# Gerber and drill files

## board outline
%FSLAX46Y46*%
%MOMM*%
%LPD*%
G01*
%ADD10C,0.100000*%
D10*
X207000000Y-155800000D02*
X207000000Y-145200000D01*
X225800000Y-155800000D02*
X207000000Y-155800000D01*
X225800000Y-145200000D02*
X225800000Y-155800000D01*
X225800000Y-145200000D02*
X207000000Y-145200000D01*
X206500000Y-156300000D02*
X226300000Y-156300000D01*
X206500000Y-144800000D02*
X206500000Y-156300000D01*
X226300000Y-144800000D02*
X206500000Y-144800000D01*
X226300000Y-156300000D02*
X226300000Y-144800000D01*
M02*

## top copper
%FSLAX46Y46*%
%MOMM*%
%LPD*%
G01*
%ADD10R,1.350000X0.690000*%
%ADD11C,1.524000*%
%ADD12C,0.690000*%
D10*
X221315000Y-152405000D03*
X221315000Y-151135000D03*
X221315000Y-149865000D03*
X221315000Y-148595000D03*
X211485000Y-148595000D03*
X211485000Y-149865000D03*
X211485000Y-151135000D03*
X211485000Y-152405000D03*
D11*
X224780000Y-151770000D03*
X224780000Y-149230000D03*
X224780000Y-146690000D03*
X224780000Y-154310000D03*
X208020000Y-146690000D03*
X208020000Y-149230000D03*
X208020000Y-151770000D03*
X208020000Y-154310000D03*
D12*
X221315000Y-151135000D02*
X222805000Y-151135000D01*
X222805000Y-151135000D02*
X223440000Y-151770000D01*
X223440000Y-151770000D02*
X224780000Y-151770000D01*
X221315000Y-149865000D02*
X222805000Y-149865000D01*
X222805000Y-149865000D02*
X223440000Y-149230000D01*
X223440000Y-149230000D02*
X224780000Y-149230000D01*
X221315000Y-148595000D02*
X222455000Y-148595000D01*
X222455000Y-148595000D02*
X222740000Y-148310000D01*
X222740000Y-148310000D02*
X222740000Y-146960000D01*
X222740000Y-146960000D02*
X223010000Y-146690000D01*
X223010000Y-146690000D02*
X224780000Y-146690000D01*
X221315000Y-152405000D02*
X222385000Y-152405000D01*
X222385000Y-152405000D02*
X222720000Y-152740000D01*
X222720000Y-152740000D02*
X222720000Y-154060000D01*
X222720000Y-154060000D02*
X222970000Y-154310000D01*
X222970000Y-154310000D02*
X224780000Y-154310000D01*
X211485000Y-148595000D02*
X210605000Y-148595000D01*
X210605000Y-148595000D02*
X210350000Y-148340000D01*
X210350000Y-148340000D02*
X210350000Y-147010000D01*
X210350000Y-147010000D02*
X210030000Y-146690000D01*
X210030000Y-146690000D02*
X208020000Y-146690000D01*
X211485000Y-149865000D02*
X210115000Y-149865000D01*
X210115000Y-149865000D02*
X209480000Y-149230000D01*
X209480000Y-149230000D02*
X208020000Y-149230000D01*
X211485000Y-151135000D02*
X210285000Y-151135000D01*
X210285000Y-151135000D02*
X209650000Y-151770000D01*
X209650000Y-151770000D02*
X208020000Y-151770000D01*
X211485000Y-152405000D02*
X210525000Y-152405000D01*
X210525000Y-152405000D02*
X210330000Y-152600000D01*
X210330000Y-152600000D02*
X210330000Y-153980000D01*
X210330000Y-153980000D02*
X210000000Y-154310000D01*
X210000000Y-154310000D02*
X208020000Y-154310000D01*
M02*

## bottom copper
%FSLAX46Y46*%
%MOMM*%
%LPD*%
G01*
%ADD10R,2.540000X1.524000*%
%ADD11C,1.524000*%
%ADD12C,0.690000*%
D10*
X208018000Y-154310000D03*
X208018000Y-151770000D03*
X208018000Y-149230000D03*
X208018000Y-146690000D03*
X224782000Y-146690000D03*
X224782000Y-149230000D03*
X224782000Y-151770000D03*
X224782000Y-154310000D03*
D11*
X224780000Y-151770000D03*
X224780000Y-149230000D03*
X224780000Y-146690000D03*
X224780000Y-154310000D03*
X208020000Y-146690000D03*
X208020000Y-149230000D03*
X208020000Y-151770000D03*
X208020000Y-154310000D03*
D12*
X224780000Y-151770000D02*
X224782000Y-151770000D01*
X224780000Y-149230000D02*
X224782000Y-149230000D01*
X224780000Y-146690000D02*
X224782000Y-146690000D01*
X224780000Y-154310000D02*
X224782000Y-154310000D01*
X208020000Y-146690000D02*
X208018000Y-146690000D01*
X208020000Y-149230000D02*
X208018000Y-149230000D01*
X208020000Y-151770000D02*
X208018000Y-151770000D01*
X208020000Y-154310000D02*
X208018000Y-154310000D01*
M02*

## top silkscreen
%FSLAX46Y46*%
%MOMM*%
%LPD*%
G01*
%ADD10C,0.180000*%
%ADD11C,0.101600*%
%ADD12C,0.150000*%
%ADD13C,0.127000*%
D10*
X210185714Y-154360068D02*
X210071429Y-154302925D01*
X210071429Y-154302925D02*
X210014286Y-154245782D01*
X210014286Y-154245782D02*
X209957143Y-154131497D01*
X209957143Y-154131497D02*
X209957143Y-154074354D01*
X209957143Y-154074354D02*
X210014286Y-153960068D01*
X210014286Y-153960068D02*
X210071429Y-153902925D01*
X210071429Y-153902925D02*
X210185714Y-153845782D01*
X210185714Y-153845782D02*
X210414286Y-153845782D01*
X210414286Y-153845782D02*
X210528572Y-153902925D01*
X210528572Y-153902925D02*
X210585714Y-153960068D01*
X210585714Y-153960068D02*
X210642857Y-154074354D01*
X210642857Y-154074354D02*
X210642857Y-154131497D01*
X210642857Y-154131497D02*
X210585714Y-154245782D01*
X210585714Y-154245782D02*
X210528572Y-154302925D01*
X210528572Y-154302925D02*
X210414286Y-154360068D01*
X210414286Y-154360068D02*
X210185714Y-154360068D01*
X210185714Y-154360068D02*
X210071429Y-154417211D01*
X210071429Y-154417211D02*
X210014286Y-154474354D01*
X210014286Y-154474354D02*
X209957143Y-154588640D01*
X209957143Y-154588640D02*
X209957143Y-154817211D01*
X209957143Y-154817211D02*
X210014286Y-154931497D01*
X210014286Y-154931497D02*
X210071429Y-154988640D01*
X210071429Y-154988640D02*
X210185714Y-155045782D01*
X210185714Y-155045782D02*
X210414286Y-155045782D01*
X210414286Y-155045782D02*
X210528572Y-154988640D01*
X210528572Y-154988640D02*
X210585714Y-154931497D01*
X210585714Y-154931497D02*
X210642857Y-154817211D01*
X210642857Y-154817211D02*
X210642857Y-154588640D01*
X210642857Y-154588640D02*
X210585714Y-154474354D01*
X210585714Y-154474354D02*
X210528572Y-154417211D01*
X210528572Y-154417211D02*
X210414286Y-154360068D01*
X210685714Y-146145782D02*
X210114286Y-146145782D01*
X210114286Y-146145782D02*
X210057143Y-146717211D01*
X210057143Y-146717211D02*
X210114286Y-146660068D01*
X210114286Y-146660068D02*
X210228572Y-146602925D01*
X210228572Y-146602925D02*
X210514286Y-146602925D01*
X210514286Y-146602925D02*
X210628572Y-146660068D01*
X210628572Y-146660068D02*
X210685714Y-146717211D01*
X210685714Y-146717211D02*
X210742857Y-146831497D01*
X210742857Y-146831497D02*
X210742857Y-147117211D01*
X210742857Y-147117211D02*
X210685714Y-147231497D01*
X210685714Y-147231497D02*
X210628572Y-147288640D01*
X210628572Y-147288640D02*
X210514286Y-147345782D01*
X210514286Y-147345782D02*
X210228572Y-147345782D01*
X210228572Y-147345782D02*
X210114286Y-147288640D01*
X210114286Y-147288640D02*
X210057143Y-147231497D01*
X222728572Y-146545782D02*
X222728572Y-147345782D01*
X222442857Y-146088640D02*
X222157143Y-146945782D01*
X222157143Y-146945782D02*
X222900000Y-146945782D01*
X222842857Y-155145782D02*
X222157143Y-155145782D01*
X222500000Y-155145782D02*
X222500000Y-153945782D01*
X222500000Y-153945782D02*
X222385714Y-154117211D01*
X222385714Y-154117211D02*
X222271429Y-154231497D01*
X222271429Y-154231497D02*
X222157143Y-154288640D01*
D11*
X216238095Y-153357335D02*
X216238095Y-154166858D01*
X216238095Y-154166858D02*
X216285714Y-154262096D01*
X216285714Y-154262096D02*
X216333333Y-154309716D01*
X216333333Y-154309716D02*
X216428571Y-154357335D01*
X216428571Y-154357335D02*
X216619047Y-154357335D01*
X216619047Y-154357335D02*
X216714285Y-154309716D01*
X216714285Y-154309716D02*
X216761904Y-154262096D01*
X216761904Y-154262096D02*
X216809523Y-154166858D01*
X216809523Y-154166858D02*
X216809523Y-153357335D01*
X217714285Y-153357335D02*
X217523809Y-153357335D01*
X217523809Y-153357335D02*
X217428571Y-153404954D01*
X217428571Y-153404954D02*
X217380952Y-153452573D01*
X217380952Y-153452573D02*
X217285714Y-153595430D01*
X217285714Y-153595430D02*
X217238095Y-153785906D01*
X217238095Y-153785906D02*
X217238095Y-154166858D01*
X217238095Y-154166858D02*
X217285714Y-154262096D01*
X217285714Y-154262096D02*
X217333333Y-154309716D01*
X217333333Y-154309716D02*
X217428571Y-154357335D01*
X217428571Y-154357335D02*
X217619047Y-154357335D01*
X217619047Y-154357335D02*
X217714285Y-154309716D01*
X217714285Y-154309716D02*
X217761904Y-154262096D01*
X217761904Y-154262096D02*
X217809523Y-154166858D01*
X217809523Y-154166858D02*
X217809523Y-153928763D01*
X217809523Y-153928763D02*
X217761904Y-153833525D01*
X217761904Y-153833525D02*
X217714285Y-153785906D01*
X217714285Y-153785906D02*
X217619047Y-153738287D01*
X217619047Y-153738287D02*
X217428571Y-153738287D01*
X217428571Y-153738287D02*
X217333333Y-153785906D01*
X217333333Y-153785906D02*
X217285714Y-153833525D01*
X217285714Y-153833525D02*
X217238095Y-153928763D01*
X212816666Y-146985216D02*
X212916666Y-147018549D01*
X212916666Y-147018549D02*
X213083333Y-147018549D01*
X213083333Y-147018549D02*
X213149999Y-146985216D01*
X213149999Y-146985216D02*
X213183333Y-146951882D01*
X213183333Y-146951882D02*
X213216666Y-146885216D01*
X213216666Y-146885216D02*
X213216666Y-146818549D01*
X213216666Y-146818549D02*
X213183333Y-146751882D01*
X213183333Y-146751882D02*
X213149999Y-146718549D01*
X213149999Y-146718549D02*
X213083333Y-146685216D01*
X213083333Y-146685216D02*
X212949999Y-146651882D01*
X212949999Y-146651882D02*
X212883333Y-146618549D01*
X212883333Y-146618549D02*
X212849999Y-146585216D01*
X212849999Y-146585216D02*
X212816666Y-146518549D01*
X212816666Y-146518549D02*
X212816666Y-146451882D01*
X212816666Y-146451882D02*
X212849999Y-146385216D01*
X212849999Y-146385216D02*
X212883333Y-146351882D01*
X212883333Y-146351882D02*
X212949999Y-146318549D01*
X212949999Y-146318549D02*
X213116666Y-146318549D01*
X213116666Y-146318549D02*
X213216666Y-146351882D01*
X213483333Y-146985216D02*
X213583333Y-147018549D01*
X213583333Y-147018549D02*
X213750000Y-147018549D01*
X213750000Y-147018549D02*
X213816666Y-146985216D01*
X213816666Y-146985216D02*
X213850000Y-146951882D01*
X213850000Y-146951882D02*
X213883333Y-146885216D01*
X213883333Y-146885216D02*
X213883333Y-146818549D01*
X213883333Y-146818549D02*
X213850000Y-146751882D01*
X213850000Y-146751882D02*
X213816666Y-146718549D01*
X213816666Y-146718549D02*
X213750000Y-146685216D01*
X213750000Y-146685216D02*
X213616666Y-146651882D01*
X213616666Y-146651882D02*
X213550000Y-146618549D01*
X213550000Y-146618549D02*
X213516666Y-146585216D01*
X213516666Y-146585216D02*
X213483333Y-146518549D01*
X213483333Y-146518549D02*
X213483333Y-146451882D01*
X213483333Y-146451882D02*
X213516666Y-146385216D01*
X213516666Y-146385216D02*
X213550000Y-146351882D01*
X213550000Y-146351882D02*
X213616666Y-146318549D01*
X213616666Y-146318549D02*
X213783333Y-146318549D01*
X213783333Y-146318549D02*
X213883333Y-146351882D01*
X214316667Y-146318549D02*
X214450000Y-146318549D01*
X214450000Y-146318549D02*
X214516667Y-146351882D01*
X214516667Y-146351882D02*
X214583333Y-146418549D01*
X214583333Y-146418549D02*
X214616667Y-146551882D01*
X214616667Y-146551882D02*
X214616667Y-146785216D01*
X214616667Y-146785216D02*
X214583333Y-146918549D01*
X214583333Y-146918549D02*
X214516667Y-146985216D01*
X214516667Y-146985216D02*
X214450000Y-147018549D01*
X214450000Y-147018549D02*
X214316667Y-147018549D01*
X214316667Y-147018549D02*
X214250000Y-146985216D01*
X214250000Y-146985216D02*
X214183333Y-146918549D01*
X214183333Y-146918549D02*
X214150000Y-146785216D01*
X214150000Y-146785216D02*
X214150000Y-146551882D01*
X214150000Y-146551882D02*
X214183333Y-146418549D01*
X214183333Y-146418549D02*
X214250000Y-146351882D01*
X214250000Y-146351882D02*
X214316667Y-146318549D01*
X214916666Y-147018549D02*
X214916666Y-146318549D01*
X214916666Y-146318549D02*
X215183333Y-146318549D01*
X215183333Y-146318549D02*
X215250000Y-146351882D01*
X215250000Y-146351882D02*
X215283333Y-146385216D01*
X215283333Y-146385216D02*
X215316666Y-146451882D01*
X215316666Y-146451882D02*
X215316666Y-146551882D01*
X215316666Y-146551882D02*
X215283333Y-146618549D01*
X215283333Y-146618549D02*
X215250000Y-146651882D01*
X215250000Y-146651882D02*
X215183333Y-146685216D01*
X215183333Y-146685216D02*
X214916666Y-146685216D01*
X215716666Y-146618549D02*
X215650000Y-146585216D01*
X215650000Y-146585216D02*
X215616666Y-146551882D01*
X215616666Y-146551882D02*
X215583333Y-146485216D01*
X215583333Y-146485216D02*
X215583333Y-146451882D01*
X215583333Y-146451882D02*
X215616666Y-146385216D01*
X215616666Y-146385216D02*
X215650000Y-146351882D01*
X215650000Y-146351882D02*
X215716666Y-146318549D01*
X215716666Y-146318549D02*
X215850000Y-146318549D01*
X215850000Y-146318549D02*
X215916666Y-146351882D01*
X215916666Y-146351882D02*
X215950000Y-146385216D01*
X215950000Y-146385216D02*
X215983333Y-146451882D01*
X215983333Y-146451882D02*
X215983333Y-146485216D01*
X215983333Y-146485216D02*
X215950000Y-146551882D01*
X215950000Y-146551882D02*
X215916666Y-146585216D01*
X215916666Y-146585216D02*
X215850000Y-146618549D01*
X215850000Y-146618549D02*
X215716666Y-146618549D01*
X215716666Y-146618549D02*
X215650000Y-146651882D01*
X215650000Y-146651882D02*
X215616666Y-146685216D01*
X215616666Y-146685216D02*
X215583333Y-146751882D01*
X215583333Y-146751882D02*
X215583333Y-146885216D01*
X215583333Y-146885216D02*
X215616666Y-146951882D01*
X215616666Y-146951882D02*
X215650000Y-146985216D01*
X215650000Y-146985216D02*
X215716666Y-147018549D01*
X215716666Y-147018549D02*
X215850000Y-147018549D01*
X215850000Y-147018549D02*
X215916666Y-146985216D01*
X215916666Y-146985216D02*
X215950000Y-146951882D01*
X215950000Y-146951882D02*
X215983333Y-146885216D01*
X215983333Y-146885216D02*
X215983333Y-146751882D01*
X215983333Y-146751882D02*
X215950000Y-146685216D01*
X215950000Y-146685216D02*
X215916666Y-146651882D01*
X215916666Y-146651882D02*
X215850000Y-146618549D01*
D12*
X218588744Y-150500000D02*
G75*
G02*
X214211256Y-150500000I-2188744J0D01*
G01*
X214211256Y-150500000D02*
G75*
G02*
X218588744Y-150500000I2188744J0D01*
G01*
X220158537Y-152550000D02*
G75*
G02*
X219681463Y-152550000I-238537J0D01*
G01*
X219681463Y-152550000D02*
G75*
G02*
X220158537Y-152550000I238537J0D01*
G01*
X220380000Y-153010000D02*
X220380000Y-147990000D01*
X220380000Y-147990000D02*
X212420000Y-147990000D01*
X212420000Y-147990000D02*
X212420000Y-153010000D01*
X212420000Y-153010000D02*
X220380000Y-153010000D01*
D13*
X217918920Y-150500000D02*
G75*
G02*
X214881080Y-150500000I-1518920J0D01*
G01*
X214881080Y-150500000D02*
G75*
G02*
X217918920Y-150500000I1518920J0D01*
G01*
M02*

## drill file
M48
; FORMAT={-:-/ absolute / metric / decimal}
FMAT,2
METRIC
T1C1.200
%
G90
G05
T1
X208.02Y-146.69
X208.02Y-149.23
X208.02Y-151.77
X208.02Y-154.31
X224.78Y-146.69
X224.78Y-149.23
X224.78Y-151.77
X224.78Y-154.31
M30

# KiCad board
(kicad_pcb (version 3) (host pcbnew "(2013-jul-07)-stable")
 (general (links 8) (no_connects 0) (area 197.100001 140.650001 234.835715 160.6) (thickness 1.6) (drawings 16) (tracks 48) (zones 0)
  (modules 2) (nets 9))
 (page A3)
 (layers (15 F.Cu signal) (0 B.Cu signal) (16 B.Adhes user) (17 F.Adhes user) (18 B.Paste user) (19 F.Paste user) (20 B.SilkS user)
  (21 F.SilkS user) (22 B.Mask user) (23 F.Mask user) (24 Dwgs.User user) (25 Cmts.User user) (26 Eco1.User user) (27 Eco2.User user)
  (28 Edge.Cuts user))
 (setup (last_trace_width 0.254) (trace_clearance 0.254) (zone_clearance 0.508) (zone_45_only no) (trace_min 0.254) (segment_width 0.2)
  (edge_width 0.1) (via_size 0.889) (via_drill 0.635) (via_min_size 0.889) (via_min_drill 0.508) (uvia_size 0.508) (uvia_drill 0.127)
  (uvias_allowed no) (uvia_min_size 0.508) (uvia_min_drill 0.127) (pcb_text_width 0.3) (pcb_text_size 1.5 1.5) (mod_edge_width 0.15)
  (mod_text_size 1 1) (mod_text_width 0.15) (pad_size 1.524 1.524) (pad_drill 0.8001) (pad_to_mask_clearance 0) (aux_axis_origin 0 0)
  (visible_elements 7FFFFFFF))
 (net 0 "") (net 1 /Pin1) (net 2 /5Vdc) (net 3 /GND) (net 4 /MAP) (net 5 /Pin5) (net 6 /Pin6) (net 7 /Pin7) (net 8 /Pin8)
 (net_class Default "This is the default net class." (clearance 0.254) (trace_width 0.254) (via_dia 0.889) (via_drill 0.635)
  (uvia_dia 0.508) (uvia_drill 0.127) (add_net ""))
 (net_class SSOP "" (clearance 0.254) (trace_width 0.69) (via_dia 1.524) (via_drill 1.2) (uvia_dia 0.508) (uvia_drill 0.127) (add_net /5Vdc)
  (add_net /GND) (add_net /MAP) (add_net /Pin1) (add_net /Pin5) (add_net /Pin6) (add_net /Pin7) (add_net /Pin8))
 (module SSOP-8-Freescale (layer F.Cu) (at 216.4 150.5)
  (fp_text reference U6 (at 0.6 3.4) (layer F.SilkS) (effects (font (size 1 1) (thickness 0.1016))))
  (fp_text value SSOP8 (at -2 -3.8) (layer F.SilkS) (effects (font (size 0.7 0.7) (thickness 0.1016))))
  (fp_circle (center 0 0) (end 2.15 0.41) (layer F.SilkS) (width 0.15))
  (fp_circle (center 3.52 2.05) (end 3.32 1.92) (layer F.SilkS) (width 0.15))
  (fp_line (start 3.98 2.51) (end 3.98 -2.51) (layer F.SilkS) (width 0.15))
  (fp_line (start 3.98 -2.51) (end -3.98 -2.51) (layer F.SilkS) (width 0.15))
  (fp_line (start -3.98 -2.51) (end -3.98 2.51) (layer F.SilkS) (width 0.15))
  (fp_line (start -3.98 2.51) (end 3.98 2.51) (layer F.SilkS) (width 0.15))
  (fp_circle (center 0 0) (end 1.51892 0) (layer F.SilkS) (width 0.127))
  (pad 1 smd rect (at 4.915 1.905) (size 1.35 0.69) (layers F.Cu F.Paste F.Mask) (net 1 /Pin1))
  (pad 2 smd rect (at 4.915 0.635) (size 1.35 0.69) (layers F.Cu F.Paste F.Mask) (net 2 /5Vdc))
  (pad 3 smd rect (at 4.915 -0.635) (size 1.35 0.69) (layers F.Cu F.Paste F.Mask) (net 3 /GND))
  (pad 4 smd rect (at 4.915 -1.905) (size 1.35 0.69) (layers F.Cu F.Paste F.Mask) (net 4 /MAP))
  (pad 5 smd rect (at -4.915 -1.905) (size 1.35 0.69) (layers F.Cu F.Paste F.Mask) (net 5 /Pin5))
  (pad 6 smd rect (at -4.915 -0.635) (size 1.35 0.69) (layers F.Cu F.Paste F.Mask) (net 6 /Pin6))
  (pad 7 smd rect (at -4.915 0.635) (size 1.35 0.69) (layers F.Cu F.Paste F.Mask) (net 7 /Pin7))
  (pad 8 smd rect (at -4.915 1.905) (size 1.35 0.69) (layers F.Cu F.Paste F.Mask) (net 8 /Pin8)))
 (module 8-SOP (layer B.Cu) (at 216.4 150.5 180)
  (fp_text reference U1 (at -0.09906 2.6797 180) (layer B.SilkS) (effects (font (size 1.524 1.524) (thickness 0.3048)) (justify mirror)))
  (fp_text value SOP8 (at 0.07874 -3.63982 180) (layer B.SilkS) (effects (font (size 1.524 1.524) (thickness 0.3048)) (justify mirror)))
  (pad 1 smd rect (at 8.382 -3.81 180) (size 2.54 1.524) (layers B.Cu B.Paste B.Mask) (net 8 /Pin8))
  (pad 2 smd rect (at 8.382 -1.27 180) (size 2.54 1.524) (layers B.Cu B.Paste B.Mask) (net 7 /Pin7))
  (pad 3 smd rect (at 8.382 1.27 180) (size 2.54 1.524) (layers B.Cu B.Paste B.Mask) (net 6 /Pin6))
  (pad 4 smd rect (at 8.382 3.81 180) (size 2.54 1.524) (layers B.Cu B.Paste B.Mask) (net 5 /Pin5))
  (pad 5 smd rect (at -8.382 3.81 180) (size 2.54 1.524) (layers B.Cu B.Paste B.Mask) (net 4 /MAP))
  (pad 6 smd rect (at -8.382 1.27 180) (size 2.54 1.524) (layers B.Cu B.Paste B.Mask) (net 3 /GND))
  (pad 7 smd rect (at -8.382 -1.27 180) (size 2.54 1.524) (layers B.Cu B.Paste B.Mask) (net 2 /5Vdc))
  (pad 8 smd rect (at -8.382 -3.81 180) (size 2.54 1.524) (layers B.Cu B.Paste B.Mask) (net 1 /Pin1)))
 (gr_line (start 207 155.8) (end 207 145.2) (angle 90) (layer Edge.Cuts) (width 0.1))
 (gr_line (start 225.8 155.8) (end 207 155.8) (angle 90) (layer Edge.Cuts) (width 0.1))
 (gr_line (start 225.8 145.2) (end 225.8 155.8) (angle 90) (layer Edge.Cuts) (width 0.1))
 (gr_line (start 225.8 145.2) (end 207 145.2) (angle 90) (layer Edge.Cuts) (width 0.1))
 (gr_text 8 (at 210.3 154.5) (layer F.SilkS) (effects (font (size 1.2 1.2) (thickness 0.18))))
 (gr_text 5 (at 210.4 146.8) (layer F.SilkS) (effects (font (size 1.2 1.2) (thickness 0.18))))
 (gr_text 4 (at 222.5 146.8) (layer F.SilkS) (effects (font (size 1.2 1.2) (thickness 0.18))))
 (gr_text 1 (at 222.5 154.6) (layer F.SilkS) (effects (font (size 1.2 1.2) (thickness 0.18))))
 (gr_line (start 206.5 156.3) (end 226.3 156.3) (angle 90) (layer Edge.Cuts) (width 0.1))
 (gr_line (start 206.5 144.8) (end 206.5 156.3) (angle 90) (layer Edge.Cuts) (width 0.1))
 (gr_line (start 226.3 144.8) (end 206.5 144.8) (angle 90) (layer Edge.Cuts) (width 0.1))
 (gr_line (start 226.3 156.3) (end 226.3 144.8) (angle 90) (layer Edge.Cuts) (width 0.1))
 (segment (start 221.315 151.135) (end 222.805 151.135) (width 0.69) (layer F.Cu) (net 2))
 (segment (start 222.805 151.135) (end 223.44 151.77) (width 0.69) (layer F.Cu) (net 2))
 (segment (start 223.44 151.77) (end 224.78 151.77) (width 0.69) (layer F.Cu) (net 2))
 (via (at 224.78 151.77) (size 1.524) (layers F.Cu B.Cu) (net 2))
 (segment (start 224.78 151.77) (end 224.782 151.77) (width 0.69) (layer B.Cu) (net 2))
 (segment (start 221.315 149.865) (end 222.805 149.865) (width 0.69) (layer F.Cu) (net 3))
 (segment (start 222.805 149.865) (end 223.44 149.23) (width 0.69) (layer F.Cu) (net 3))
 (segment (start 223.44 149.23) (end 224.78 149.23) (width 0.69) (layer F.Cu) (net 3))
 (via (at 224.78 149.23) (size 1.524) (layers F.Cu B.Cu) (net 3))
 (segment (start 224.78 149.23) (end 224.782 149.23) (width 0.69) (layer B.Cu) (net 3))
 (segment (start 221.315 148.595) (end 222.455 148.595) (width 0.69) (layer F.Cu) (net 4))
 (segment (start 222.455 148.595) (end 222.74 148.31) (width 0.69) (layer F.Cu) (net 4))
 (segment (start 222.74 148.31) (end 222.74 146.96) (width 0.69) (layer F.Cu) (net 4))
 (segment (start 222.74 146.96) (end 223.01 146.69) (width 0.69) (layer F.Cu) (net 4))
 (segment (start 223.01 146.69) (end 224.78 146.69) (width 0.69) (layer F.Cu) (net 4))
 (via (at 224.78 146.69) (size 1.524) (layers F.Cu B.Cu) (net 4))
 (segment (start 224.78 146.69) (end 224.782 146.69) (width 0.69) (layer B.Cu) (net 4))
 (segment (start 221.315 152.405) (end 222.385 152.405) (width 0.69) (layer F.Cu) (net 1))
 (segment (start 222.385 152.405) (end 222.72 152.74) (width 0.69) (layer F.Cu) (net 1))
 (segment (start 222.72 152.74) (end 222.72 154.06) (width 0.69) (layer F.Cu) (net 1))
 (segment (start 222.72 154.06) (end 222.97 154.31) (width 0.69) (layer F.Cu) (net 1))
 (segment (start 222.97 154.31) (end 224.78 154.31) (width 0.69) (layer F.Cu) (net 1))
 (via (at 224.78 154.31) (size 1.524) (layers F.Cu B.Cu) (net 1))
 (segment (start 224.78 154.31) (end 224.782 154.31) (width 0.69) (layer B.Cu) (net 1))
 (segment (start 211.485 148.595) (end 210.605 148.595) (width 0.69) (layer F.Cu) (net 5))
 (segment (start 210.605 148.595) (end 210.35 148.34) (width 0.69) (layer F.Cu) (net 5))
 (segment (start 210.35 148.34) (end 210.35 147.01) (width 0.69) (layer F.Cu) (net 5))
 (segment (start 210.35 147.01) (end 210.03 146.69) (width 0.69) (layer F.Cu) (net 5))
 (segment (start 210.03 146.69) (end 208.02 146.69) (width 0.69) (layer F.Cu) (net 5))
 (via (at 208.02 146.69) (size 1.524) (layers F.Cu B.Cu) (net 5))
 (segment (start 208.02 146.69) (end 208.018 146.69) (width 0.69) (layer B.Cu) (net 5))
 (segment (start 211.485 149.865) (end 210.115 149.865) (width 0.69) (layer F.Cu) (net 6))
 (segment (start 210.115 149.865) (end 209.48 149.23) (width 0.69) (layer F.Cu) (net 6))
 (segment (start 209.48 149.23) (end 208.02 149.23) (width 0.69) (layer F.Cu) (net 6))
 (via (at 208.02 149.23) (size 1.524) (layers F.Cu B.Cu) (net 6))
 (segment (start 208.02 149.23) (end 208.018 149.23) (width 0.69) (layer B.Cu) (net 6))
 (segment (start 211.485 151.135) (end 210.285 151.135) (width 0.69) (layer F.Cu) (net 7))
 (segment (start 210.285 151.135) (end 209.65 151.77) (width 0.69) (layer F.Cu) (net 7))
 (segment (start 209.65 151.77) (end 208.02 151.77) (width 0.69) (layer F.Cu) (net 7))
 (via (at 208.02 151.77) (size 1.524) (layers F.Cu B.Cu) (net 7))
 (segment (start 208.02 151.77) (end 208.018 151.77) (width 0.69) (layer B.Cu) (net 7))
 (segment (start 211.485 152.405) (end 210.525 152.405) (width 0.69) (layer F.Cu) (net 8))
 (segment (start 210.525 152.405) (end 210.33 152.6) (width 0.69) (layer F.Cu) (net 8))
 (segment (start 210.33 152.6) (end 210.33 153.98) (width 0.69) (layer F.Cu) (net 8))
 (segment (start 210.33 153.98) (end 210 154.31) (width 0.69) (layer F.Cu) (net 8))
 (segment (start 210 154.31) (end 208.02 154.31) (width 0.69) (layer F.Cu) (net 8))
 (via (at 208.02 154.31) (size 1.524) (layers F.Cu B.Cu) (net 8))
 (segment (start 208.02 154.31) (end 208.018 154.31) (width 0.69) (layer B.Cu) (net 8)))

